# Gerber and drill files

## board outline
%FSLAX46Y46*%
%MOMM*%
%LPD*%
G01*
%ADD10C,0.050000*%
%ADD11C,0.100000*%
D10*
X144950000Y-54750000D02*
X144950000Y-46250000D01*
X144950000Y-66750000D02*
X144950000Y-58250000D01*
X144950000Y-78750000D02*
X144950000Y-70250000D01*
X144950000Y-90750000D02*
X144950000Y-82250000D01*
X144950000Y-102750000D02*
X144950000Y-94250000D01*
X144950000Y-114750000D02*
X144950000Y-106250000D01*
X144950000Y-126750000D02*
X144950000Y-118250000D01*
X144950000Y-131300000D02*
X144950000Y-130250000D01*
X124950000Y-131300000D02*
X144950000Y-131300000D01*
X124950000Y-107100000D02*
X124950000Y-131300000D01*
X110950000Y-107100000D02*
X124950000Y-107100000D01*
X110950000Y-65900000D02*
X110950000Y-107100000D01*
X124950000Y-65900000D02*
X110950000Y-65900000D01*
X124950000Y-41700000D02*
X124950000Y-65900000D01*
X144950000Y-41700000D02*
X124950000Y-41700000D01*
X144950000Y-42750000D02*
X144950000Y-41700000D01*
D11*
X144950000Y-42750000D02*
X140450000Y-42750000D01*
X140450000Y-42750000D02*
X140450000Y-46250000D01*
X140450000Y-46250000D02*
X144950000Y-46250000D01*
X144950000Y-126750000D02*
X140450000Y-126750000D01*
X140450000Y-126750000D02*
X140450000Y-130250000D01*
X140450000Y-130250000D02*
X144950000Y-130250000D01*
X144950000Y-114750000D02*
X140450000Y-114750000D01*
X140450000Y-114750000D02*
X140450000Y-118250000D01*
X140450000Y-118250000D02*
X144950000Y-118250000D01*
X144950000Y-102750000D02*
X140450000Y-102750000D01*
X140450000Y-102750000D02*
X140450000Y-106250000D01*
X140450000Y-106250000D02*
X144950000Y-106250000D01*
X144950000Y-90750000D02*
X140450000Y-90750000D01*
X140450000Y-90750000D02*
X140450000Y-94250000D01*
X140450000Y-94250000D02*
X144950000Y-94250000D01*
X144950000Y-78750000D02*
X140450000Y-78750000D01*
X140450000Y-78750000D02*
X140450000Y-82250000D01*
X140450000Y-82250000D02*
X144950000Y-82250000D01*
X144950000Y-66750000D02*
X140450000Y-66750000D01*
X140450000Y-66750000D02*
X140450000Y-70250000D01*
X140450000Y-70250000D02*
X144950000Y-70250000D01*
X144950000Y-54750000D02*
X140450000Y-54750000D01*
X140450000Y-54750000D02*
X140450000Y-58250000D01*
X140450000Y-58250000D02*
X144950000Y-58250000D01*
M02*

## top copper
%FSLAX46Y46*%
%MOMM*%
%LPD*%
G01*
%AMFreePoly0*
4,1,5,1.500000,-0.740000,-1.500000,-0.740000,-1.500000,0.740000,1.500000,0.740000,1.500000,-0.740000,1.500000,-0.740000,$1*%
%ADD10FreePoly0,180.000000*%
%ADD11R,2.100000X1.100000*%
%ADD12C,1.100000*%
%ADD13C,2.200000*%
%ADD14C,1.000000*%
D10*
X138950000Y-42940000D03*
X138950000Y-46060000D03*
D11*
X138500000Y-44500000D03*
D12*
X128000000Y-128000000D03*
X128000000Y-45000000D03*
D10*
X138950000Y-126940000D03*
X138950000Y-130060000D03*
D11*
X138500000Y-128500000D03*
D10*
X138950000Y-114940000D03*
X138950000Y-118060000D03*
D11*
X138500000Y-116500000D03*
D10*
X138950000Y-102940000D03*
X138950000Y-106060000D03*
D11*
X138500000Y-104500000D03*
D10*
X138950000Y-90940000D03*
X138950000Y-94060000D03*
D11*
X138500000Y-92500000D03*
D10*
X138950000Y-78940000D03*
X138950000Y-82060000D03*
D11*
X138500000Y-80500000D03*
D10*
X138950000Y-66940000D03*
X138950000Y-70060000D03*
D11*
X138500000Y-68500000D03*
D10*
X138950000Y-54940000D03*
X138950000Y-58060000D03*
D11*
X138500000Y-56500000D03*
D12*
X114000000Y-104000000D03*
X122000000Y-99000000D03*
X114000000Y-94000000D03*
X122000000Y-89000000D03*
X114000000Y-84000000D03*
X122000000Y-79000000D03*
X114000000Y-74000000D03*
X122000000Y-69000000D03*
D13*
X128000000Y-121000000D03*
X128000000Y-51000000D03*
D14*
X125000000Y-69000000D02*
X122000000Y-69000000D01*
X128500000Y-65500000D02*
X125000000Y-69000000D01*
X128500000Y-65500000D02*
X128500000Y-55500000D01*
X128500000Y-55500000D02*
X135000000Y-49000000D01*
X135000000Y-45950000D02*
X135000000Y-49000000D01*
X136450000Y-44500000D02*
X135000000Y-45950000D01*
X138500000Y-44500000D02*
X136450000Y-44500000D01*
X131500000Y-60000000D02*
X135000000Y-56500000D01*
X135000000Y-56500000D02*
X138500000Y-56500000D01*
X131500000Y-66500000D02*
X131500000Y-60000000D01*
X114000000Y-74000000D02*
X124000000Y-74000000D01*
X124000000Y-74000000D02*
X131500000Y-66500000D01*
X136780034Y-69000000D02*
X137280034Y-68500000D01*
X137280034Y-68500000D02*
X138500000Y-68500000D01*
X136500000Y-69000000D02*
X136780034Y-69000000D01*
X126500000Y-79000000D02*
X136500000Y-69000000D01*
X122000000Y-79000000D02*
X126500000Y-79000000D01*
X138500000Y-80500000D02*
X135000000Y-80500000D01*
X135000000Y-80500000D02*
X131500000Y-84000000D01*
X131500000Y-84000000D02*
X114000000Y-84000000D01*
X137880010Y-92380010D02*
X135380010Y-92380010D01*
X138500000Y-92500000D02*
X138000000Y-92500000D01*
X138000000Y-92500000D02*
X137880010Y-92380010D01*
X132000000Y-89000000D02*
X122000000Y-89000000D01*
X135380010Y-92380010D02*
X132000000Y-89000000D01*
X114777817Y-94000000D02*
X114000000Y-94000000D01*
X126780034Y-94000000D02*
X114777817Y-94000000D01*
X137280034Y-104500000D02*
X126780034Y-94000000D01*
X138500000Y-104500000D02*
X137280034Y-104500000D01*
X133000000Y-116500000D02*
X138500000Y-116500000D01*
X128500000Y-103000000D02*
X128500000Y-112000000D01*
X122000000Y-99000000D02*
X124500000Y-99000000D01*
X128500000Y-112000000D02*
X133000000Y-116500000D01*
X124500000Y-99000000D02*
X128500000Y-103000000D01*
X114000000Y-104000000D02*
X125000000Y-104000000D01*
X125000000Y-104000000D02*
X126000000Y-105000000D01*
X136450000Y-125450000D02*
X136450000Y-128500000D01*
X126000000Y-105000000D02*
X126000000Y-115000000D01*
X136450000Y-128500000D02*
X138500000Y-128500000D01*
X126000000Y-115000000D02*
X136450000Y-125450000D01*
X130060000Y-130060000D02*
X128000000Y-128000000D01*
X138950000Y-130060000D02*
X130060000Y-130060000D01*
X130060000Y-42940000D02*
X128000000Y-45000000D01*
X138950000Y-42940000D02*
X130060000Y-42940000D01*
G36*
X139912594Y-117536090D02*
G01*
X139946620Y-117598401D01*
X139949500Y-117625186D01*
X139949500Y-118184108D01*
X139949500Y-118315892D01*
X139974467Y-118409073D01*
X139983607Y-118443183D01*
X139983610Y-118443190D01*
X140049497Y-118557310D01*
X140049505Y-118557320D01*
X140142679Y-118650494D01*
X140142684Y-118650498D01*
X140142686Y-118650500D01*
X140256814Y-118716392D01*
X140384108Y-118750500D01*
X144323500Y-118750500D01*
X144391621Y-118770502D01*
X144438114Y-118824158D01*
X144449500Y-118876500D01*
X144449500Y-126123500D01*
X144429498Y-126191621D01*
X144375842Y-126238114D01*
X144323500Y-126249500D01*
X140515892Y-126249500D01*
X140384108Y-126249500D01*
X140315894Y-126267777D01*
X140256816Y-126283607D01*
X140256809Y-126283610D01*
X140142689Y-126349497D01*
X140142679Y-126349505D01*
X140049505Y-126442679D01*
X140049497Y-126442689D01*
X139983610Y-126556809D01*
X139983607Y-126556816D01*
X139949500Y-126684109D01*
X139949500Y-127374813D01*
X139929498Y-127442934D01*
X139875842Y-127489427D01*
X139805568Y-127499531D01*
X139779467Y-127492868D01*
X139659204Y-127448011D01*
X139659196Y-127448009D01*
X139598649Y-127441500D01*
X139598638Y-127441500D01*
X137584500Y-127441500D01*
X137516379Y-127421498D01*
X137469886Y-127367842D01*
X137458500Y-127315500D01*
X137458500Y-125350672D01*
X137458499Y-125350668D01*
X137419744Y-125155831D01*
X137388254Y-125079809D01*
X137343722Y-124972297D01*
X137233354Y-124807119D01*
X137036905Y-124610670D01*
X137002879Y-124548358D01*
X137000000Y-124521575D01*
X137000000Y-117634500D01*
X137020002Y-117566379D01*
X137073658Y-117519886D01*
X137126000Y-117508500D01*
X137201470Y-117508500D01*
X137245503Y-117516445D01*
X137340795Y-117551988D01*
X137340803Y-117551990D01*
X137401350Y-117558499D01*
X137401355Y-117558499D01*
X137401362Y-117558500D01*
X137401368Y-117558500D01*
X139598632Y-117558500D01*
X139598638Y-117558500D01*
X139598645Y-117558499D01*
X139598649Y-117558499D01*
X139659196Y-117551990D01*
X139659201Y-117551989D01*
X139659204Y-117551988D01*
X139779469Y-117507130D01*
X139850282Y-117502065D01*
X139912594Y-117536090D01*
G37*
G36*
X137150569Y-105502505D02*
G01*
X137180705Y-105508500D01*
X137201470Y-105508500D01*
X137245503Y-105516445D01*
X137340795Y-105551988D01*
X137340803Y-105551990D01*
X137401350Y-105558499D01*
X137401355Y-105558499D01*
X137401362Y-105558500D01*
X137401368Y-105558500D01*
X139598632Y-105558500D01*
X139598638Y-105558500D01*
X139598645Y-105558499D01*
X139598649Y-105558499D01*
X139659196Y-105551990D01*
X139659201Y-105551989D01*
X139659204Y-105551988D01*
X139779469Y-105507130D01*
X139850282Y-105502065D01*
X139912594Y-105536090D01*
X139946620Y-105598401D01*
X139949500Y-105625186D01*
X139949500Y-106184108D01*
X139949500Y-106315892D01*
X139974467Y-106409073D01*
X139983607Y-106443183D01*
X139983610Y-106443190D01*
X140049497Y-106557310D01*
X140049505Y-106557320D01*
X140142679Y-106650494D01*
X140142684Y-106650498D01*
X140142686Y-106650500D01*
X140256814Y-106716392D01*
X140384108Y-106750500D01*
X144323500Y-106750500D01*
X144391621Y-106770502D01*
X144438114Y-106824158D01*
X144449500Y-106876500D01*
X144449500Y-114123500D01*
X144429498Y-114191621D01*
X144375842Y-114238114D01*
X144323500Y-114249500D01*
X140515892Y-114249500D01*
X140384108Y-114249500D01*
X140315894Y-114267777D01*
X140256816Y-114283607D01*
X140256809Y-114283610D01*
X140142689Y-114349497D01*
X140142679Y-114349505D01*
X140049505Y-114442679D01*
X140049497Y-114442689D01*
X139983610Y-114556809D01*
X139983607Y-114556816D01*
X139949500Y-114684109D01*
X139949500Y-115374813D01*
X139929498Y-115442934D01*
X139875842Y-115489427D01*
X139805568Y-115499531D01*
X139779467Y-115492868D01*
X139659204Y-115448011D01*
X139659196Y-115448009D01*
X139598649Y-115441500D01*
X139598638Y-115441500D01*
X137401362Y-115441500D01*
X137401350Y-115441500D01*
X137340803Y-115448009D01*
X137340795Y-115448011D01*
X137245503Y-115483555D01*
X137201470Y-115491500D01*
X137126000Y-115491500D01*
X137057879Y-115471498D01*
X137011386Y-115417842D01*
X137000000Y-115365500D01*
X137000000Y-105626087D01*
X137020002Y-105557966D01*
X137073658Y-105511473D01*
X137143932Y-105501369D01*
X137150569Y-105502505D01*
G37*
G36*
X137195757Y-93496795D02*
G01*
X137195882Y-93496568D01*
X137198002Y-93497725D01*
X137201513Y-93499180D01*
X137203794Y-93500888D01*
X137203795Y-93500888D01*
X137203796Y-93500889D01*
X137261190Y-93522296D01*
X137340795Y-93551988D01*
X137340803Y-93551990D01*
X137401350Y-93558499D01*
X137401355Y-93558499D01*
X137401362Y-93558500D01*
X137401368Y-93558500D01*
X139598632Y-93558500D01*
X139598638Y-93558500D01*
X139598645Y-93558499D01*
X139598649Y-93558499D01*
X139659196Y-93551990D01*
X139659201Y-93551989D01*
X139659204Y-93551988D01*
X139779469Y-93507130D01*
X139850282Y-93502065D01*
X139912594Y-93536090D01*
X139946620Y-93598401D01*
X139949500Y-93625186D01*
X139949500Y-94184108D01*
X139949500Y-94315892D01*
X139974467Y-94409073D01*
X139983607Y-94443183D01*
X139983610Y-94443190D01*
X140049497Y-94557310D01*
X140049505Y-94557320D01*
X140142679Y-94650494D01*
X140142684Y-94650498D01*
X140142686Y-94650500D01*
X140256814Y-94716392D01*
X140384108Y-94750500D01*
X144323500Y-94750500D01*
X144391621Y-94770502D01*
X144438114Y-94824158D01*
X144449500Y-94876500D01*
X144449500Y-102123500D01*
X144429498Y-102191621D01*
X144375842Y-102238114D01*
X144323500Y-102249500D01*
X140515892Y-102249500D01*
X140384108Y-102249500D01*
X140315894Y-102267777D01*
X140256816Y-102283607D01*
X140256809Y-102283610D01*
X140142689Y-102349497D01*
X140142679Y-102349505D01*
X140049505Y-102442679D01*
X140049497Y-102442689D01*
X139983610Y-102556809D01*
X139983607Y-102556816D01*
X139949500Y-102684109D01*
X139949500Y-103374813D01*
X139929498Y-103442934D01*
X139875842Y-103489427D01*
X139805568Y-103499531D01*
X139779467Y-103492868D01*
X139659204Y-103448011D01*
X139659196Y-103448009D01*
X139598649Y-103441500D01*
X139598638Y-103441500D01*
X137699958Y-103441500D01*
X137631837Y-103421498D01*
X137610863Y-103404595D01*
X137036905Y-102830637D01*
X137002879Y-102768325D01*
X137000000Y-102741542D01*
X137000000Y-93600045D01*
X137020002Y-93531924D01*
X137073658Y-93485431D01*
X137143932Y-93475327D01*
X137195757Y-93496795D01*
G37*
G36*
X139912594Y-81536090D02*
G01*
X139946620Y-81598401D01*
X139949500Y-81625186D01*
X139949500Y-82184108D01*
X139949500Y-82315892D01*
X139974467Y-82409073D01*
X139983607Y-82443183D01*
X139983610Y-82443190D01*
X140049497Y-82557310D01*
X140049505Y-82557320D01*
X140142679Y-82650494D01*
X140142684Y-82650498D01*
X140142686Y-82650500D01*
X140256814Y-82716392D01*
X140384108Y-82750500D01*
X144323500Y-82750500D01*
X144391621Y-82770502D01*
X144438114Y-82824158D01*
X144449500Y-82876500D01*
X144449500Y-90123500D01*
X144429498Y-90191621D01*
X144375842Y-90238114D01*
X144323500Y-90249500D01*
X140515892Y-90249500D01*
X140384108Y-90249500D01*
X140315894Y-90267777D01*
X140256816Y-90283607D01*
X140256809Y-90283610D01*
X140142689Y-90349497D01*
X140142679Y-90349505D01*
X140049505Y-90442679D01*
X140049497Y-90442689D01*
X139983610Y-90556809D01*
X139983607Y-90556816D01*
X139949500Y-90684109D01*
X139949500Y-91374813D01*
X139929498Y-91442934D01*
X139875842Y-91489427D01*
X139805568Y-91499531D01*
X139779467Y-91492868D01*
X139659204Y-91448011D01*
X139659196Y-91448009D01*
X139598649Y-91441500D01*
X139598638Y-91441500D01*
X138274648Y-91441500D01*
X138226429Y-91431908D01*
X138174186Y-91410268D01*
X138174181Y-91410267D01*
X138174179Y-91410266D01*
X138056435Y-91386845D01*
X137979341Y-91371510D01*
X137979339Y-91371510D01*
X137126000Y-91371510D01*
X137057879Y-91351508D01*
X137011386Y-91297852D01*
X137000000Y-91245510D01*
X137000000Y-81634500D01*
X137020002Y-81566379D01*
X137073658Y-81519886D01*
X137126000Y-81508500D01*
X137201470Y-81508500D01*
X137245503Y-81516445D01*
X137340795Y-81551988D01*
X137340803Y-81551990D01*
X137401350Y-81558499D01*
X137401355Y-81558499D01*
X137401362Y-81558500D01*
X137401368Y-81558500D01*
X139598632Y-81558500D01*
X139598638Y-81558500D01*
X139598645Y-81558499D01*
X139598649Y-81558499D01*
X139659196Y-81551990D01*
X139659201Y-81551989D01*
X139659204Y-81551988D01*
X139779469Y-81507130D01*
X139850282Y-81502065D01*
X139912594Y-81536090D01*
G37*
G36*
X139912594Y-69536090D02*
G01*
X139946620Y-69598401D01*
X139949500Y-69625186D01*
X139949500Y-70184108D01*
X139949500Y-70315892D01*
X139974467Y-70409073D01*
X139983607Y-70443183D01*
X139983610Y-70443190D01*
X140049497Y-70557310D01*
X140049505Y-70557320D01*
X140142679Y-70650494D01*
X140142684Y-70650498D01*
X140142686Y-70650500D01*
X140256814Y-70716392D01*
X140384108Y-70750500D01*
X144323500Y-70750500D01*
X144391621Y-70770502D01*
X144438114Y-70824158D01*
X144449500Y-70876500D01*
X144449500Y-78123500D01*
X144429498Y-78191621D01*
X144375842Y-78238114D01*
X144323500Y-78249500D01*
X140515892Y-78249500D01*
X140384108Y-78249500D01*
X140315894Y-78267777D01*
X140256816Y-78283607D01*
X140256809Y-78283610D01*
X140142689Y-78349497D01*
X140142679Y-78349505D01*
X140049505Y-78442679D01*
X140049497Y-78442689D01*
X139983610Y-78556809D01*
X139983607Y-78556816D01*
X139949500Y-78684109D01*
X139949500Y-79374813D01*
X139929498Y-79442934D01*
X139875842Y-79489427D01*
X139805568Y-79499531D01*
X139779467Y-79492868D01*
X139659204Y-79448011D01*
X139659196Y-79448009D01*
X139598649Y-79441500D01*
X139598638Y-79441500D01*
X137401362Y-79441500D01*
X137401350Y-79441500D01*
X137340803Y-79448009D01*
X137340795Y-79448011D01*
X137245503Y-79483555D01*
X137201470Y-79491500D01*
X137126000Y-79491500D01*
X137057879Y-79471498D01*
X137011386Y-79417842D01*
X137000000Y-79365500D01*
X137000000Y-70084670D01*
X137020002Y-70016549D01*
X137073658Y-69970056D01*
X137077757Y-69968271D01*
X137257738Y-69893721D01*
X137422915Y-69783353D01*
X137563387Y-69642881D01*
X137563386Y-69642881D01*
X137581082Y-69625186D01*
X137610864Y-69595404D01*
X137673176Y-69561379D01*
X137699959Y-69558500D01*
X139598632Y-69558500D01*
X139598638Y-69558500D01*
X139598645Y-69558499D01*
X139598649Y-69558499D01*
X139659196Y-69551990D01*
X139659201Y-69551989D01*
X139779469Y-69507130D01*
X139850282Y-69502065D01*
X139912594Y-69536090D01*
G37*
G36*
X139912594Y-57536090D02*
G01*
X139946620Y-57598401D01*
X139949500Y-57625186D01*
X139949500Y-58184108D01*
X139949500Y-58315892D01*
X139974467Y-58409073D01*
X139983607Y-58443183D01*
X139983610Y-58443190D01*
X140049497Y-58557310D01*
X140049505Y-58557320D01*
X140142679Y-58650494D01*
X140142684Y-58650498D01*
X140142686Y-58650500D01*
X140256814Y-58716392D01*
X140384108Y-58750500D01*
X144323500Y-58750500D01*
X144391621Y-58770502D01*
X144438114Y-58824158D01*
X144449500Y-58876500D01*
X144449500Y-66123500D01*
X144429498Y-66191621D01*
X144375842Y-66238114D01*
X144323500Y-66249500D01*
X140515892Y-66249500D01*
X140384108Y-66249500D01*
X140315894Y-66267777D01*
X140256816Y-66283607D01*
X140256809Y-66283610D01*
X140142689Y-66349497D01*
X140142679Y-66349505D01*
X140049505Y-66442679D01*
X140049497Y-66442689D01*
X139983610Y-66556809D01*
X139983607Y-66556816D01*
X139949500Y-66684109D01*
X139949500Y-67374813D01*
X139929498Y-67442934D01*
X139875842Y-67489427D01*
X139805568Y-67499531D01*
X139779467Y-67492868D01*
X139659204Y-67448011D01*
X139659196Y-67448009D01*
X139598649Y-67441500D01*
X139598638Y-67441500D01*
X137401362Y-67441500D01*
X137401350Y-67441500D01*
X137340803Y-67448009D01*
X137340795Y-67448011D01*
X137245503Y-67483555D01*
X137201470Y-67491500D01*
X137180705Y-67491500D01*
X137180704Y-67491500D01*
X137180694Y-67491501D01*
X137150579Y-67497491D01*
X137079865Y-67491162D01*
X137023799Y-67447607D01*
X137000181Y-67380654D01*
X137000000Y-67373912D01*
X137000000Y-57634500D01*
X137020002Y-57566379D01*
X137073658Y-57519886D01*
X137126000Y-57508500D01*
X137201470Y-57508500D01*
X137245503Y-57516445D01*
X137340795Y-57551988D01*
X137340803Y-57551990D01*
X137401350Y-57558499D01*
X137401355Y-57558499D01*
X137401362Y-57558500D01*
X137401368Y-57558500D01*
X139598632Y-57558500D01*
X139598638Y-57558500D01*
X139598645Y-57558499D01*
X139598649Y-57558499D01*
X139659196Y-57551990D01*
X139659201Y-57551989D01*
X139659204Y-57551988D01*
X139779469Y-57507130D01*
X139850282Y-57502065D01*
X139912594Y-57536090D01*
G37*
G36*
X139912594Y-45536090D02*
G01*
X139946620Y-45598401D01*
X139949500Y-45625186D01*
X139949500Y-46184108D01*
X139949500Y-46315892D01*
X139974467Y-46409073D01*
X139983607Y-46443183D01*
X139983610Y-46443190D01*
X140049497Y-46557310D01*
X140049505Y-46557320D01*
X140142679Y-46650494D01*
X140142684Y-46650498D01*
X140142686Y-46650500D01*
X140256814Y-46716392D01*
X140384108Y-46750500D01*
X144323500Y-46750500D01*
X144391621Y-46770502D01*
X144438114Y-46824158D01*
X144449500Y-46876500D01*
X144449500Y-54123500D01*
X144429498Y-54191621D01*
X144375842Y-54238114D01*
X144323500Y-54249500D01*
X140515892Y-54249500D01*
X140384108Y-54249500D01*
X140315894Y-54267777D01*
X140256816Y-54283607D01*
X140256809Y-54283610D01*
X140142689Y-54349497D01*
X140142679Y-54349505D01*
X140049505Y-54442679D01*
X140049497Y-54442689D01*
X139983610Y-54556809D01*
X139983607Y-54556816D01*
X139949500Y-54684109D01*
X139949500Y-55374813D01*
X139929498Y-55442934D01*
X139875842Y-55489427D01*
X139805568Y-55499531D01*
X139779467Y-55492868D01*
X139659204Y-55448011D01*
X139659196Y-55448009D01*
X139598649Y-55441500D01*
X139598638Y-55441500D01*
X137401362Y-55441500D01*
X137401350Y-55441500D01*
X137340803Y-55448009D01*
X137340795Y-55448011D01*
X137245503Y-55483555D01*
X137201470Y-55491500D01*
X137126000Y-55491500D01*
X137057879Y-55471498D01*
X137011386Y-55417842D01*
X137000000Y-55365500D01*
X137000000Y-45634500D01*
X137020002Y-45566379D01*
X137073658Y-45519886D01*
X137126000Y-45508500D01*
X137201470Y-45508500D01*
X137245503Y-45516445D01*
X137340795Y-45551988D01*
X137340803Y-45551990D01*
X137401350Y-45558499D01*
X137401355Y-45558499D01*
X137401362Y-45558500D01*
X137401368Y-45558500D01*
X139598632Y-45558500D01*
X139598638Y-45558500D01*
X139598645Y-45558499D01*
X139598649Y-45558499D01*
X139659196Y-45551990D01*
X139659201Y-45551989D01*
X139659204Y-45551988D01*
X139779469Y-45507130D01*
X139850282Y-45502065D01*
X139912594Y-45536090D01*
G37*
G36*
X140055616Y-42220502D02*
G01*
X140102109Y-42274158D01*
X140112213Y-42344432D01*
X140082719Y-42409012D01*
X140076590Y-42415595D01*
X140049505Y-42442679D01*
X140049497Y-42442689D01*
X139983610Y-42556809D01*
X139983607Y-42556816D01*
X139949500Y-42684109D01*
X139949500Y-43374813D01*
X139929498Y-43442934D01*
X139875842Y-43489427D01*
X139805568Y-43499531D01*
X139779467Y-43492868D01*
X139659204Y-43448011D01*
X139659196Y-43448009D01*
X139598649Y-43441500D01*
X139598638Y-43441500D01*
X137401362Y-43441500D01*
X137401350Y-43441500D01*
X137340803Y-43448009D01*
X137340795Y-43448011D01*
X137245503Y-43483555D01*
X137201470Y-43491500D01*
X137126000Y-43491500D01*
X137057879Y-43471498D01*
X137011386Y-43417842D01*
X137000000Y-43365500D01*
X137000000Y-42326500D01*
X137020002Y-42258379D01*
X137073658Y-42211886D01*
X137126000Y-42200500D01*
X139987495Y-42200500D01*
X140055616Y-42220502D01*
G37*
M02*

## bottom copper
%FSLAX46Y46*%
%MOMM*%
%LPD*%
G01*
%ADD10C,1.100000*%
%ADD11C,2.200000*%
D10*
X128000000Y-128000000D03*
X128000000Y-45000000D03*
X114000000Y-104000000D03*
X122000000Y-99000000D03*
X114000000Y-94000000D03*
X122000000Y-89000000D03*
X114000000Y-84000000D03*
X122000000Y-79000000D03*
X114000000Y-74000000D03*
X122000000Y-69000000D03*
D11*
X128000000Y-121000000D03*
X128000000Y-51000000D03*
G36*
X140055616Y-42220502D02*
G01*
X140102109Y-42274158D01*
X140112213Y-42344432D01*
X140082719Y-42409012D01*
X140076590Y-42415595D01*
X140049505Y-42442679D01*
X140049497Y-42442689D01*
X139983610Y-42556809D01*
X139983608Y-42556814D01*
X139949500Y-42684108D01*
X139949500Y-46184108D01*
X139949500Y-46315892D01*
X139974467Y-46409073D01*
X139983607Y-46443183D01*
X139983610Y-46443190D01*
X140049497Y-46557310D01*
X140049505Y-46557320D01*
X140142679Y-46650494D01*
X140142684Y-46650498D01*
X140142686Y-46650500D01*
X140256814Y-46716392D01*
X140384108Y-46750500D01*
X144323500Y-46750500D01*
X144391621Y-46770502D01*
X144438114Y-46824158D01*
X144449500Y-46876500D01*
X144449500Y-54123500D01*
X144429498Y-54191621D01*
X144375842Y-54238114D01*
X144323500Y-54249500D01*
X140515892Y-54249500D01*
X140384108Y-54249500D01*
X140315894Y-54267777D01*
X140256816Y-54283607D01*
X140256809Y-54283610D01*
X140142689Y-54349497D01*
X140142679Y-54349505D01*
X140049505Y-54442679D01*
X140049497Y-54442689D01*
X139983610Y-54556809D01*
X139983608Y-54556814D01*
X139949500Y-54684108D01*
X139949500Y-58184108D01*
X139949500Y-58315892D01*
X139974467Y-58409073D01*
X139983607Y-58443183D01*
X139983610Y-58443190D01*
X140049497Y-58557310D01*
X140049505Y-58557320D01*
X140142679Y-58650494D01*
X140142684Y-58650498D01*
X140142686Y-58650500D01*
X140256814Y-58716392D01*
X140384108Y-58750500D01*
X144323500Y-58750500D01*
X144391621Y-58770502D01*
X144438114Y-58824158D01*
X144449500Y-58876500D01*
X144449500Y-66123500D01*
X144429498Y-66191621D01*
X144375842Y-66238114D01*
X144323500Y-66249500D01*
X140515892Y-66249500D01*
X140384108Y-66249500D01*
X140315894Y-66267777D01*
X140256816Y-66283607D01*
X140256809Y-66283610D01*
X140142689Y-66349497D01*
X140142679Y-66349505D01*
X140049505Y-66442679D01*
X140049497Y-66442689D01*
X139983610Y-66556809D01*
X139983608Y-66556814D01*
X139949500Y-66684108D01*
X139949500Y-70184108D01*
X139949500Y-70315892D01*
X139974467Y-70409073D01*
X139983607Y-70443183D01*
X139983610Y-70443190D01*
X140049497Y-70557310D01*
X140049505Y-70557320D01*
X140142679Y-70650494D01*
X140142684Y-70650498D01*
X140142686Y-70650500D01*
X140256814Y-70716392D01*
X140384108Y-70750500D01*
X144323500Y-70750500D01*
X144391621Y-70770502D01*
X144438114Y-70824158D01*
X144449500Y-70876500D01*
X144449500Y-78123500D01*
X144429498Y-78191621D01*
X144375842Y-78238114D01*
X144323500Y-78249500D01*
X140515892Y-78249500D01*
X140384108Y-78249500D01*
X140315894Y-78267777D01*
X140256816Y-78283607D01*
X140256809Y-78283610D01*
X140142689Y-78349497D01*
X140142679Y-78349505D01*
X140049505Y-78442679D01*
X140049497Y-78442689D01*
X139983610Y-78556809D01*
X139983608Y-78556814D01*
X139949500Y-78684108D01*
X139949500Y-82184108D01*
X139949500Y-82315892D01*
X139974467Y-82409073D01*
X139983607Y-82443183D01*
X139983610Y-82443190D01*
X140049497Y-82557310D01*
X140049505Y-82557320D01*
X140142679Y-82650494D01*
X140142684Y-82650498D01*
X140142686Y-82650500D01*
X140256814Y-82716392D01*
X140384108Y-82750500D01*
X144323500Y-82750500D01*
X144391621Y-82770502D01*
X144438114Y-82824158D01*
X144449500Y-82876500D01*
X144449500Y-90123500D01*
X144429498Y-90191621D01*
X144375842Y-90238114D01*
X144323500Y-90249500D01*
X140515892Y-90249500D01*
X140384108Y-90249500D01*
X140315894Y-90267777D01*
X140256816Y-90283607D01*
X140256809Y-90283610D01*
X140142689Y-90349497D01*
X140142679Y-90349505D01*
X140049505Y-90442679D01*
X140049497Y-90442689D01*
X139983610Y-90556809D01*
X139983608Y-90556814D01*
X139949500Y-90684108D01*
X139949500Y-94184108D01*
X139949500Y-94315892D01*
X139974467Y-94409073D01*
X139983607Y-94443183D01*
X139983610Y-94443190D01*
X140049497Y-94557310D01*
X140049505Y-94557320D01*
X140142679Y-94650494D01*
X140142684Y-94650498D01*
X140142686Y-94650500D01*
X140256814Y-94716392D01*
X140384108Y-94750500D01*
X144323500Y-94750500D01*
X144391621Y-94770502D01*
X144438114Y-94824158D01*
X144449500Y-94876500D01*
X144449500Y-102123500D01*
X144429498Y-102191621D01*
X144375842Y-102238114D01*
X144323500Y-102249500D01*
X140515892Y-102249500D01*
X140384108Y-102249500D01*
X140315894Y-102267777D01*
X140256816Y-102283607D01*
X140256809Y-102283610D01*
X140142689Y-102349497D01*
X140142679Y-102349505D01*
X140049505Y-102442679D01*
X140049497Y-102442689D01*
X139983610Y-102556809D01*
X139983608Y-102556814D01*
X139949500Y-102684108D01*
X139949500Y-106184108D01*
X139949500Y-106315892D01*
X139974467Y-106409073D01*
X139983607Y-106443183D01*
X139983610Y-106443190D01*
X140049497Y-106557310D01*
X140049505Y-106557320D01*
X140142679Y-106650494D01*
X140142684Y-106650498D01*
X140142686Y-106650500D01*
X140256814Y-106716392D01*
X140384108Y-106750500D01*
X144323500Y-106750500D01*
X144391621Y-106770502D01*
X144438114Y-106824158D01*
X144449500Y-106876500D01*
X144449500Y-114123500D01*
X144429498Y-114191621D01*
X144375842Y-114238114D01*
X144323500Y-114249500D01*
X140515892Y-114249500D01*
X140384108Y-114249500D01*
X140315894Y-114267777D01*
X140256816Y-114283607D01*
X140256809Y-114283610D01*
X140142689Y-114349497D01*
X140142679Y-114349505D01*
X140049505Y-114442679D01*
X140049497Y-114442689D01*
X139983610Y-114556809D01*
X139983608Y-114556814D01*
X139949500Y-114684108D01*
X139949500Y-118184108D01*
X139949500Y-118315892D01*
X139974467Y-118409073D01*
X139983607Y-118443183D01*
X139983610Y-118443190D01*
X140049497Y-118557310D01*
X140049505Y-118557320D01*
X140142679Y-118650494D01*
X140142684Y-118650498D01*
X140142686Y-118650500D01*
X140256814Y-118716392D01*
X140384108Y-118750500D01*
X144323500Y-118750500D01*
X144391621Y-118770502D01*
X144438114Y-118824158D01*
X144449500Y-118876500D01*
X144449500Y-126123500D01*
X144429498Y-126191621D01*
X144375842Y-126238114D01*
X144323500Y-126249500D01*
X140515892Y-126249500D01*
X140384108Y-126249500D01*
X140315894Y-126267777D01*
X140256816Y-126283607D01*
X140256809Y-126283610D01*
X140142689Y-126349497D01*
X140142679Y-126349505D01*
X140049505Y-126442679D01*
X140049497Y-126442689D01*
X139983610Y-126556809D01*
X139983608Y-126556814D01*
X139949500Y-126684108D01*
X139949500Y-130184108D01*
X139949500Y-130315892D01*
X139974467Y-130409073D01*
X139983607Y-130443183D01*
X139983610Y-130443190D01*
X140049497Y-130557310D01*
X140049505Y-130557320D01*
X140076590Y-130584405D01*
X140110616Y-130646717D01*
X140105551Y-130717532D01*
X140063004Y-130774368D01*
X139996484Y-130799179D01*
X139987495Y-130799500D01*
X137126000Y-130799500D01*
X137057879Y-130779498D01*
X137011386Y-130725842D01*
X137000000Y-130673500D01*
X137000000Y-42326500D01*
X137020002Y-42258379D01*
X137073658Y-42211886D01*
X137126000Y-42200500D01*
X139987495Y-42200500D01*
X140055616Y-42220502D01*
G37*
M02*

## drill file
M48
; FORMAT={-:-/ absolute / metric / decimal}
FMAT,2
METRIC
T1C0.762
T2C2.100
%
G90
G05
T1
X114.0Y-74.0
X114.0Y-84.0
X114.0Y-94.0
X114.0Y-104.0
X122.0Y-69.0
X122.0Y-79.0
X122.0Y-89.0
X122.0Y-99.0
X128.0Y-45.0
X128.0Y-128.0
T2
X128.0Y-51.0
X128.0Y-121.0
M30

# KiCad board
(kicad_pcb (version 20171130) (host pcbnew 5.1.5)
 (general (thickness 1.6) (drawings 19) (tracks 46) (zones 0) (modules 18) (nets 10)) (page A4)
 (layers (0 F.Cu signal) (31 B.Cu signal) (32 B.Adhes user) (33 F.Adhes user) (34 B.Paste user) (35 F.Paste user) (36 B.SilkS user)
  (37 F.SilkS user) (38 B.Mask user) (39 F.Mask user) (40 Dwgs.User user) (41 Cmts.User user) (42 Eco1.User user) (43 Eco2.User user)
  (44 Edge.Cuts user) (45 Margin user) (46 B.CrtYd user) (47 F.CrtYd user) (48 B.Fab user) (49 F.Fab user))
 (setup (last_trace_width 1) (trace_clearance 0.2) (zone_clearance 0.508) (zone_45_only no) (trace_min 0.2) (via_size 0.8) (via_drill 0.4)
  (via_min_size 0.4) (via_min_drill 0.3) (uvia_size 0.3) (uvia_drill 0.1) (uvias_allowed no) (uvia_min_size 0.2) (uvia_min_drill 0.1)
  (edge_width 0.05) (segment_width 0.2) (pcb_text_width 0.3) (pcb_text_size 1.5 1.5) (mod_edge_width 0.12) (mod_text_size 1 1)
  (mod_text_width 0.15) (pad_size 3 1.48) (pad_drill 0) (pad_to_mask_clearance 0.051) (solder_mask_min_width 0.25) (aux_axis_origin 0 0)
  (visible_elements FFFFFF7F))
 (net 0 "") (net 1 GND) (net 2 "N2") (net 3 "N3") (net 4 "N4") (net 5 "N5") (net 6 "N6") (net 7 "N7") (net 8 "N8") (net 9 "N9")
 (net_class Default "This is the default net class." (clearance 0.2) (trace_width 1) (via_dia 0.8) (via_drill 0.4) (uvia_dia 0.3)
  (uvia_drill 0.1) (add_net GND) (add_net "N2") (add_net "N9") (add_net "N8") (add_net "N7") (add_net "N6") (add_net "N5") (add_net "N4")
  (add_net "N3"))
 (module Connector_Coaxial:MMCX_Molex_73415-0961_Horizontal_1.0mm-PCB (layer F.Cu) (at 141.2 44.5 180)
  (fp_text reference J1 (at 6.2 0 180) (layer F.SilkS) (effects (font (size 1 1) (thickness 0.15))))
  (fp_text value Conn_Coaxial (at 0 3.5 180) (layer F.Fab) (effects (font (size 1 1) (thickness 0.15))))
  (fp_line (start -3.75 1.75) (end 0.75 1.75) (layer Edge.Cuts) (width 0.1))
  (fp_line (start 0.75 1.75) (end 0.75 -1.75) (layer Edge.Cuts) (width 0.1))
  (fp_line (start 0.75 -1.75) (end -3.75 -1.75) (layer Edge.Cuts) (width 0.1))
  (pad 2 smd custom (at 2.25 1.56 180) (size 3 1.48) (layers F.Cu F.Paste F.Mask) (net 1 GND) (zone_connect 2)
   (options (clearance outline) (anchor rect)) (primitives))
  (pad 2 smd custom (at 2.25 -1.56 180) (size 3 1.48) (layers F.Cu F.Paste F.Mask) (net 1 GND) (zone_connect 2)
   (options (clearance outline) (anchor rect)) (primitives))
  (pad 1 smd rect (at 2.7 0 180) (size 2.1 1.1) (layers F.Cu F.Paste F.Mask) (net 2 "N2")))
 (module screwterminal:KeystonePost (layer F.Cu) (at 128 128)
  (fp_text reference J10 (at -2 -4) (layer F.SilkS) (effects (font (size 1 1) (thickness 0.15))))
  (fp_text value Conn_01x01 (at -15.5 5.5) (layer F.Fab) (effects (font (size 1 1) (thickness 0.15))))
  (pad 1 thru_hole circle (at 0 0) (size 1.1 1.1) (drill 0.762) (layers *.Cu *.Mask) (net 1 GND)))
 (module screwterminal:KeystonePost (layer F.Cu) (at 128 45)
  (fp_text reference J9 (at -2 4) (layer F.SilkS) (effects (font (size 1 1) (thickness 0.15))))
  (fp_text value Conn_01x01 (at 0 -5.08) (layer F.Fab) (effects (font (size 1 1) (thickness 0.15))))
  (pad 1 thru_hole circle (at 0 0) (size 1.1 1.1) (drill 0.762) (layers *.Cu *.Mask) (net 1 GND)))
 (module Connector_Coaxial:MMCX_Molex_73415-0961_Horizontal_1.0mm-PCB (layer F.Cu) (at 141.2 128.5 180)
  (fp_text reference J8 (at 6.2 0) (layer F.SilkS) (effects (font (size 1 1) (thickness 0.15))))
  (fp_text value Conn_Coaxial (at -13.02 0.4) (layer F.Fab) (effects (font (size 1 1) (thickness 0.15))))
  (fp_line (start -3.75 1.75) (end 0.75 1.75) (layer Edge.Cuts) (width 0.1))
  (fp_line (start 0.75 1.75) (end 0.75 -1.75) (layer Edge.Cuts) (width 0.1))
  (fp_line (start 0.75 -1.75) (end -3.75 -1.75) (layer Edge.Cuts) (width 0.1))
  (pad 2 smd custom (at 2.25 1.56 180) (size 3 1.48) (layers F.Cu F.Paste F.Mask) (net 1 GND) (zone_connect 2)
   (options (clearance outline) (anchor rect)) (primitives))
  (pad 2 smd custom (at 2.25 -1.56 180) (size 3 1.48) (layers F.Cu F.Paste F.Mask) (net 1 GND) (options (clearance outline) (anchor rect))
   (primitives))
  (pad 1 smd rect (at 2.7 0 180) (size 2.1 1.1) (layers F.Cu F.Paste F.Mask) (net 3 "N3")))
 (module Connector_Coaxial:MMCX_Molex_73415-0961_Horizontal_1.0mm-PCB (layer F.Cu) (at 141.2 116.5 180)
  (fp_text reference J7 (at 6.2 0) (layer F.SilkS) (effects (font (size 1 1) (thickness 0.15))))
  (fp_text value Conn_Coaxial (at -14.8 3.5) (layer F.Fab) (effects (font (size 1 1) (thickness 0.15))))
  (fp_line (start -3.75 1.75) (end 0.75 1.75) (layer Edge.Cuts) (width 0.1))
  (fp_line (start 0.75 1.75) (end 0.75 -1.75) (layer Edge.Cuts) (width 0.1))
  (fp_line (start 0.75 -1.75) (end -3.75 -1.75) (layer Edge.Cuts) (width 0.1))
  (pad 2 smd custom (at 2.25 1.56 180) (size 3 1.48) (layers F.Cu F.Paste F.Mask) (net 1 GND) (zone_connect 2)
   (options (clearance outline) (anchor rect)) (primitives))
  (pad 2 smd custom (at 2.25 -1.56 180) (size 3 1.48) (layers F.Cu F.Paste F.Mask) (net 1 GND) (zone_connect 2)
   (options (clearance outline) (anchor rect)) (primitives))
  (pad 1 smd rect (at 2.7 0 180) (size 2.1 1.1) (layers F.Cu F.Paste F.Mask) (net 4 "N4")))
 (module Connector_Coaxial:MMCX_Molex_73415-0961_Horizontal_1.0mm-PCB (layer F.Cu) (at 141.2 104.5 180)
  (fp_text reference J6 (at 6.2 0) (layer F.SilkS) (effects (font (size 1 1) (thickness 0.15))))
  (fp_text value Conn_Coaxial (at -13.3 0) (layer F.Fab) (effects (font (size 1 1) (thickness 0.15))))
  (fp_line (start -3.75 1.75) (end 0.75 1.75) (layer Edge.Cuts) (width 0.1))
  (fp_line (start 0.75 1.75) (end 0.75 -1.75) (layer Edge.Cuts) (width 0.1))
  (fp_line (start 0.75 -1.75) (end -3.75 -1.75) (layer Edge.Cuts) (width 0.1))
  (pad 2 smd custom (at 2.25 1.56 180) (size 3 1.48) (layers F.Cu F.Paste F.Mask) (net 1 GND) (zone_connect 2)
   (options (clearance outline) (anchor rect)) (primitives))
  (pad 2 smd custom (at 2.25 -1.56 180) (size 3 1.48) (layers F.Cu F.Paste F.Mask) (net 1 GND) (zone_connect 2)
   (options (clearance outline) (anchor rect)) (primitives))
  (pad 1 smd rect (at 2.7 0 180) (size 2.1 1.1) (layers F.Cu F.Paste F.Mask) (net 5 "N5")))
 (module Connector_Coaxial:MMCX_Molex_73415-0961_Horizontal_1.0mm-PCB (layer F.Cu) (at 141.2 92.5 180)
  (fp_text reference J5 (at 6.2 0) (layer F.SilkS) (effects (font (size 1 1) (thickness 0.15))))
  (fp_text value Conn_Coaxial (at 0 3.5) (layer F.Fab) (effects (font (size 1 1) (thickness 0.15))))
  (fp_line (start -3.75 1.75) (end 0.75 1.75) (layer Edge.Cuts) (width 0.1))
  (fp_line (start 0.75 1.75) (end 0.75 -1.75) (layer Edge.Cuts) (width 0.1))
  (fp_line (start 0.75 -1.75) (end -3.75 -1.75) (layer Edge.Cuts) (width 0.1))
  (pad 2 smd custom (at 2.25 1.56 180) (size 3 1.48) (layers F.Cu F.Paste F.Mask) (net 1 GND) (zone_connect 2)
   (options (clearance outline) (anchor rect)) (primitives))
  (pad 2 smd custom (at 2.25 -1.56 180) (size 3 1.48) (layers F.Cu F.Paste F.Mask) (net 1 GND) (zone_connect 2)
   (options (clearance outline) (anchor rect)) (primitives))
  (pad 1 smd rect (at 2.7 0 180) (size 2.1 1.1) (layers F.Cu F.Paste F.Mask) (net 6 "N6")))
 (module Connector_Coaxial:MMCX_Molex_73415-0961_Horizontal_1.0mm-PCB (layer F.Cu) (at 141.2 80.5 180)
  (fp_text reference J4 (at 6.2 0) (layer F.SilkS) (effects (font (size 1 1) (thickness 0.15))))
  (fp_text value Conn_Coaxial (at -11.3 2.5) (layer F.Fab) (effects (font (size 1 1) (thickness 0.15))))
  (fp_line (start -3.75 1.75) (end 0.75 1.75) (layer Edge.Cuts) (width 0.1))
  (fp_line (start 0.75 1.75) (end 0.75 -1.75) (layer Edge.Cuts) (width 0.1))
  (fp_line (start 0.75 -1.75) (end -3.75 -1.75) (layer Edge.Cuts) (width 0.1))
  (pad 2 smd custom (at 2.25 1.56 180) (size 3 1.48) (layers F.Cu F.Paste F.Mask) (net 1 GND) (zone_connect 2)
   (options (clearance outline) (anchor rect)) (primitives))
  (pad 2 smd custom (at 2.25 -1.56 180) (size 3 1.48) (layers F.Cu F.Paste F.Mask) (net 1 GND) (zone_connect 2)
   (options (clearance outline) (anchor rect)) (primitives))
  (pad 1 smd rect (at 2.7 0 180) (size 2.1 1.1) (layers F.Cu F.Paste F.Mask) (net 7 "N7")))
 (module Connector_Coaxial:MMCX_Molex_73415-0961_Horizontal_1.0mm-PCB (layer F.Cu) (at 141.2 68.5 180)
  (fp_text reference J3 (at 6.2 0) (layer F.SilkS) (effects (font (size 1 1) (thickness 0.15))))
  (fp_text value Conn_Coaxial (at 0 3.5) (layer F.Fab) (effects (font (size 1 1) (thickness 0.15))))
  (fp_line (start -3.75 1.75) (end 0.75 1.75) (layer Edge.Cuts) (width 0.1))
  (fp_line (start 0.75 1.75) (end 0.75 -1.75) (layer Edge.Cuts) (width 0.1))
  (fp_line (start 0.75 -1.75) (end -3.75 -1.75) (layer Edge.Cuts) (width 0.1))
  (pad 2 smd custom (at 2.25 1.56 180) (size 3 1.48) (layers F.Cu F.Paste F.Mask) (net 1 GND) (zone_connect 2)
   (options (clearance outline) (anchor rect)) (primitives))
  (pad 2 smd custom (at 2.25 -1.56 180) (size 3 1.48) (layers F.Cu F.Paste F.Mask) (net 1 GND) (zone_connect 2)
   (options (clearance outline) (anchor rect)) (primitives))
  (pad 1 smd rect (at 2.7 0 180) (size 2.1 1.1) (layers F.Cu F.Paste F.Mask) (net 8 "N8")))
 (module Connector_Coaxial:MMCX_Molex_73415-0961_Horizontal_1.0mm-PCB (layer F.Cu) (at 141.2 56.5 180)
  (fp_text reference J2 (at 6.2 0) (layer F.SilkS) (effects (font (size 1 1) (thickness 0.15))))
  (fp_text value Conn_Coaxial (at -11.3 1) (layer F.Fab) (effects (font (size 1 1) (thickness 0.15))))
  (fp_line (start -3.75 1.75) (end 0.75 1.75) (layer Edge.Cuts) (width 0.1))
  (fp_line (start 0.75 1.75) (end 0.75 -1.75) (layer Edge.Cuts) (width 0.1))
  (fp_line (start 0.75 -1.75) (end -3.75 -1.75) (layer Edge.Cuts) (width 0.1))
  (pad 2 smd custom (at 2.25 1.56 180) (size 3 1.48) (layers F.Cu F.Paste F.Mask) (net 1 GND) (zone_connect 2)
   (options (clearance outline) (anchor rect)) (primitives))
  (pad 2 smd custom (at 2.25 -1.56 180) (size 3 1.48) (layers F.Cu F.Paste F.Mask) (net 1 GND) (zone_connect 2)
   (options (clearance outline) (anchor rect)) (primitives))
  (pad 1 smd rect (at 2.7 0 180) (size 2.1 1.1) (layers F.Cu F.Paste F.Mask) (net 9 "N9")))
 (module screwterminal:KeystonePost (layer F.Cu) (at 114 104)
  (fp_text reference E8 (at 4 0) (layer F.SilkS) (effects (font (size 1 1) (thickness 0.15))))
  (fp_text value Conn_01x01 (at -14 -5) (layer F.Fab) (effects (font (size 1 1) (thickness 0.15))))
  (pad 1 thru_hole circle (at 0 0) (size 1.1 1.1) (drill 0.762) (layers *.Cu *.Mask) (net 3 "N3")))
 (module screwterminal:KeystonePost (layer F.Cu) (at 122 99)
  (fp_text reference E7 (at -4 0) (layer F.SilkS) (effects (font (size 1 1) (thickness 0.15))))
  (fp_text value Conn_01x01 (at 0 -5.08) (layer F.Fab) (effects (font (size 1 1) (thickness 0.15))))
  (pad 1 thru_hole circle (at 0 0) (size 1.1 1.1) (drill 0.762) (layers *.Cu *.Mask) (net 4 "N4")))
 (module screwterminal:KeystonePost (layer F.Cu) (at 114 94)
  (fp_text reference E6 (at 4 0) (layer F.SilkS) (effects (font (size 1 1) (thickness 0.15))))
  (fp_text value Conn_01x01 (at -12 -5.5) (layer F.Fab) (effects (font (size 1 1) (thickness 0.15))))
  (pad 1 thru_hole circle (at 0 0) (size 1.1 1.1) (drill 0.762) (layers *.Cu *.Mask) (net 5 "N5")))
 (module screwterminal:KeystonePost (layer F.Cu) (at 122 89)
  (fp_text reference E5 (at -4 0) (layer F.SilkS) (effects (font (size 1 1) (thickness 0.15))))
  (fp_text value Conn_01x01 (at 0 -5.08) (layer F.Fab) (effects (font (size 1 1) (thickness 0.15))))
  (pad 1 thru_hole circle (at 0 0) (size 1.1 1.1) (drill 0.762) (layers *.Cu *.Mask) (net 6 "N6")))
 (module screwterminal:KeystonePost (layer F.Cu) (at 114 84)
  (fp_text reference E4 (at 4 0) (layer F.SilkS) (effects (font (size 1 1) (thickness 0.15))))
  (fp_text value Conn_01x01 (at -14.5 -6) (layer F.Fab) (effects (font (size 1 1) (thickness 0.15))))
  (pad 1 thru_hole circle (at 0 0) (size 1.1 1.1) (drill 0.762) (layers *.Cu *.Mask) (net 7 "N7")))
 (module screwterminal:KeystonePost (layer F.Cu) (at 122 79)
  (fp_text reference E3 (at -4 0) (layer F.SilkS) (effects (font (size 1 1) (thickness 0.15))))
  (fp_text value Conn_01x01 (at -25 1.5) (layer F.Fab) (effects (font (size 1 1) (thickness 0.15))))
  (pad 1 thru_hole circle (at 0 0) (size 1.1 1.1) (drill 0.762) (layers *.Cu *.Mask) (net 8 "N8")))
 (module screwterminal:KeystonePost (layer F.Cu) (at 114 74)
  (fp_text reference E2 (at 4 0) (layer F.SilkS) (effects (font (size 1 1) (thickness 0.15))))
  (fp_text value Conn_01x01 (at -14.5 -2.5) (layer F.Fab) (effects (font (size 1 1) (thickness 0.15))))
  (pad 1 thru_hole circle (at 0 0) (size 1.1 1.1) (drill 0.762) (layers *.Cu *.Mask) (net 9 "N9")))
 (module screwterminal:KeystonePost (layer F.Cu) (at 122 69)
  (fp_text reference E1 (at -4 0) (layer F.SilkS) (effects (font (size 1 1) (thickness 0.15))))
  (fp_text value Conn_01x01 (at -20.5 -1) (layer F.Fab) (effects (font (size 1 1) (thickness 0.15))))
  (pad 1 thru_hole circle (at 0 0) (size 1.1 1.1) (drill 0.762) (layers *.Cu *.Mask) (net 2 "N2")))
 (gr_line (start 144.95 54.75) (end 144.95 46.25) (layer Edge.Cuts) (width 0.05))
 (gr_line (start 144.95 66.75) (end 144.95 58.25) (layer Edge.Cuts) (width 0.05))
 (gr_line (start 144.95 78.75) (end 144.95 70.25) (layer Edge.Cuts) (width 0.05))
 (gr_line (start 144.95 90.75) (end 144.95 82.25) (layer Edge.Cuts) (width 0.05))
 (gr_line (start 144.95 102.75) (end 144.95 94.25) (layer Edge.Cuts) (width 0.05))
 (gr_line (start 144.95 114.75) (end 144.95 106.25) (layer Edge.Cuts) (width 0.05))
 (gr_line (start 144.95 126.75) (end 144.95 118.25) (layer Edge.Cuts) (width 0.05))
 (gr_line (start 144.95 131.3) (end 144.95 130.25) (layer Edge.Cuts) (width 0.05))
 (gr_line (start 124.95 131.3) (end 144.95 131.3) (layer Edge.Cuts) (width 0.05))
 (gr_line (start 124.95 107.1) (end 124.95 131.3) (layer Edge.Cuts) (width 0.05))
 (gr_line (start 110.95 107.1) (end 124.95 107.1) (layer Edge.Cuts) (width 0.05))
 (gr_line (start 110.95 65.9) (end 110.95 107.1) (layer Edge.Cuts) (width 0.05))
 (gr_line (start 124.95 65.9) (end 110.95 65.9) (layer Edge.Cuts) (width 0.05))
 (gr_line (start 124.95 41.7) (end 124.95 65.9) (layer Edge.Cuts) (width 0.05))
 (gr_line (start 144.95 41.7) (end 124.95 41.7) (layer Edge.Cuts) (width 0.05))
 (gr_line (start 144.95 42.75) (end 144.95 41.7) (layer Edge.Cuts) (width 0.05))
 (via (at 128 121) (size 2.2) (drill 2.1) (layers F.Cu B.Cu) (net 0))
 (via (at 128 51) (size 2.2) (drill 2.1) (layers F.Cu B.Cu) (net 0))
 (segment (start 125 69) (end 122 69) (width 1) (layer F.Cu) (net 2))
 (segment (start 128.5 65.5) (end 125 69) (width 1) (layer F.Cu) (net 2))
 (segment (start 128.5 65.5) (end 128.5 55.5) (width 1) (layer F.Cu) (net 2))
 (segment (start 128.5 55.5) (end 135 49) (width 1) (layer F.Cu) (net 2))
 (segment (start 135 45.95) (end 135 49) (width 1) (layer F.Cu) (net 2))
 (segment (start 136.45 44.5) (end 135 45.95) (width 1) (layer F.Cu) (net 2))
 (segment (start 138.5 44.5) (end 136.45 44.5) (width 1) (layer F.Cu) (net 2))
 (segment (start 131.5 60) (end 135 56.5) (width 1) (layer F.Cu) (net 9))
 (segment (start 135 56.5) (end 138.5 56.5) (width 1) (layer F.Cu) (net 9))
 (segment (start 131.5 66.5) (end 131.5 60) (width 1) (layer F.Cu) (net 9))
 (segment (start 114 74) (end 124 74) (width 1) (layer F.Cu) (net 9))
 (segment (start 124 74) (end 131.5 66.5) (width 1) (layer F.Cu) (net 9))
 (segment (start 136.780034 69) (end 137.280034 68.5) (width 1) (layer F.Cu) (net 8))
 (segment (start 137.280034 68.5) (end 138.5 68.5) (width 1) (layer F.Cu) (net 8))
 (segment (start 136.5 69) (end 136.780034 69) (width 1) (layer F.Cu) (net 8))
 (segment (start 126.5 79) (end 136.5 69) (width 1) (layer F.Cu) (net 8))
 (segment (start 122 79) (end 126.5 79) (width 1) (layer F.Cu) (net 8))
 (segment (start 138.5 80.5) (end 135 80.5) (width 1) (layer F.Cu) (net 7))
 (segment (start 135 80.5) (end 131.5 84) (width 1) (layer F.Cu) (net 7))
 (segment (start 131.5 84) (end 114 84) (width 1) (layer F.Cu) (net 7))
 (segment (start 137.88001 92.38001) (end 135.38001 92.38001) (width 1) (layer F.Cu) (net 6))
 (segment (start 138.5 92.5) (end 138 92.5) (width 1) (layer F.Cu) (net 6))
 (segment (start 138 92.5) (end 137.88001 92.38001) (width 1) (layer F.Cu) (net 6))
 (segment (start 132 89) (end 122 89) (width 1) (layer F.Cu) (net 6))
 (segment (start 135.38001 92.38001) (end 132 89) (width 1) (layer F.Cu) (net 6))
 (segment (start 114.777817 94) (end 114 94) (width 1) (layer F.Cu) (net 5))
 (segment (start 126.780034 94) (end 114.777817 94) (width 1) (layer F.Cu) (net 5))
 (segment (start 137.280034 104.5) (end 126.780034 94) (width 1) (layer F.Cu) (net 5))
 (segment (start 138.5 104.5) (end 137.280034 104.5) (width 1) (layer F.Cu) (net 5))
 (segment (start 133 116.5) (end 138.5 116.5) (width 1) (layer F.Cu) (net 4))
 (segment (start 128.5 103) (end 128.5 112) (width 1) (layer F.Cu) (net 4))
 (segment (start 122 99) (end 124.5 99) (width 1) (layer F.Cu) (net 4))
 (segment (start 128.5 112) (end 133 116.5) (width 1) (layer F.Cu) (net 4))
 (segment (start 124.5 99) (end 128.5 103) (width 1) (layer F.Cu) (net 4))
 (segment (start 114 104) (end 125 104) (width 1) (layer F.Cu) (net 3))
 (segment (start 125 104) (end 126 105) (width 1) (layer F.Cu) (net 3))
 (segment (start 136.45 125.45) (end 136.45 128.5) (width 1) (layer F.Cu) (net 3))
 (segment (start 126 105) (end 126 115) (width 1) (layer F.Cu) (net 3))
 (segment (start 136.45 128.5) (end 138.5 128.5) (width 1) (layer F.Cu) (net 3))
 (segment (start 126 115) (end 136.45 125.45) (width 1) (layer F.Cu) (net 3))
 (segment (start 130.06 130.06) (end 128 128) (width 1) (layer F.Cu) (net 1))
 (segment (start 138.95 130.06) (end 130.06 130.06) (width 1) (layer F.Cu) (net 1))
 (segment (start 130.06 42.94) (end 128 45) (width 1) (layer F.Cu) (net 1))
 (segment (start 138.95 42.94) (end 130.06 42.94) (width 1) (layer F.Cu) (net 1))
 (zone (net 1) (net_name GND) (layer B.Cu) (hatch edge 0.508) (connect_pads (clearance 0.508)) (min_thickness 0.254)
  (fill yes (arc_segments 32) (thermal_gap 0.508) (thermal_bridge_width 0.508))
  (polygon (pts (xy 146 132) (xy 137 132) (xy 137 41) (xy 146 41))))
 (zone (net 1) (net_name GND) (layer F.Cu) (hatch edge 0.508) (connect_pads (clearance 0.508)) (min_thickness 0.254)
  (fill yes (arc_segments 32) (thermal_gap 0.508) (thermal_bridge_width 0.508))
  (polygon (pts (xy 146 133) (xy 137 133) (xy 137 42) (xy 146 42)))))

